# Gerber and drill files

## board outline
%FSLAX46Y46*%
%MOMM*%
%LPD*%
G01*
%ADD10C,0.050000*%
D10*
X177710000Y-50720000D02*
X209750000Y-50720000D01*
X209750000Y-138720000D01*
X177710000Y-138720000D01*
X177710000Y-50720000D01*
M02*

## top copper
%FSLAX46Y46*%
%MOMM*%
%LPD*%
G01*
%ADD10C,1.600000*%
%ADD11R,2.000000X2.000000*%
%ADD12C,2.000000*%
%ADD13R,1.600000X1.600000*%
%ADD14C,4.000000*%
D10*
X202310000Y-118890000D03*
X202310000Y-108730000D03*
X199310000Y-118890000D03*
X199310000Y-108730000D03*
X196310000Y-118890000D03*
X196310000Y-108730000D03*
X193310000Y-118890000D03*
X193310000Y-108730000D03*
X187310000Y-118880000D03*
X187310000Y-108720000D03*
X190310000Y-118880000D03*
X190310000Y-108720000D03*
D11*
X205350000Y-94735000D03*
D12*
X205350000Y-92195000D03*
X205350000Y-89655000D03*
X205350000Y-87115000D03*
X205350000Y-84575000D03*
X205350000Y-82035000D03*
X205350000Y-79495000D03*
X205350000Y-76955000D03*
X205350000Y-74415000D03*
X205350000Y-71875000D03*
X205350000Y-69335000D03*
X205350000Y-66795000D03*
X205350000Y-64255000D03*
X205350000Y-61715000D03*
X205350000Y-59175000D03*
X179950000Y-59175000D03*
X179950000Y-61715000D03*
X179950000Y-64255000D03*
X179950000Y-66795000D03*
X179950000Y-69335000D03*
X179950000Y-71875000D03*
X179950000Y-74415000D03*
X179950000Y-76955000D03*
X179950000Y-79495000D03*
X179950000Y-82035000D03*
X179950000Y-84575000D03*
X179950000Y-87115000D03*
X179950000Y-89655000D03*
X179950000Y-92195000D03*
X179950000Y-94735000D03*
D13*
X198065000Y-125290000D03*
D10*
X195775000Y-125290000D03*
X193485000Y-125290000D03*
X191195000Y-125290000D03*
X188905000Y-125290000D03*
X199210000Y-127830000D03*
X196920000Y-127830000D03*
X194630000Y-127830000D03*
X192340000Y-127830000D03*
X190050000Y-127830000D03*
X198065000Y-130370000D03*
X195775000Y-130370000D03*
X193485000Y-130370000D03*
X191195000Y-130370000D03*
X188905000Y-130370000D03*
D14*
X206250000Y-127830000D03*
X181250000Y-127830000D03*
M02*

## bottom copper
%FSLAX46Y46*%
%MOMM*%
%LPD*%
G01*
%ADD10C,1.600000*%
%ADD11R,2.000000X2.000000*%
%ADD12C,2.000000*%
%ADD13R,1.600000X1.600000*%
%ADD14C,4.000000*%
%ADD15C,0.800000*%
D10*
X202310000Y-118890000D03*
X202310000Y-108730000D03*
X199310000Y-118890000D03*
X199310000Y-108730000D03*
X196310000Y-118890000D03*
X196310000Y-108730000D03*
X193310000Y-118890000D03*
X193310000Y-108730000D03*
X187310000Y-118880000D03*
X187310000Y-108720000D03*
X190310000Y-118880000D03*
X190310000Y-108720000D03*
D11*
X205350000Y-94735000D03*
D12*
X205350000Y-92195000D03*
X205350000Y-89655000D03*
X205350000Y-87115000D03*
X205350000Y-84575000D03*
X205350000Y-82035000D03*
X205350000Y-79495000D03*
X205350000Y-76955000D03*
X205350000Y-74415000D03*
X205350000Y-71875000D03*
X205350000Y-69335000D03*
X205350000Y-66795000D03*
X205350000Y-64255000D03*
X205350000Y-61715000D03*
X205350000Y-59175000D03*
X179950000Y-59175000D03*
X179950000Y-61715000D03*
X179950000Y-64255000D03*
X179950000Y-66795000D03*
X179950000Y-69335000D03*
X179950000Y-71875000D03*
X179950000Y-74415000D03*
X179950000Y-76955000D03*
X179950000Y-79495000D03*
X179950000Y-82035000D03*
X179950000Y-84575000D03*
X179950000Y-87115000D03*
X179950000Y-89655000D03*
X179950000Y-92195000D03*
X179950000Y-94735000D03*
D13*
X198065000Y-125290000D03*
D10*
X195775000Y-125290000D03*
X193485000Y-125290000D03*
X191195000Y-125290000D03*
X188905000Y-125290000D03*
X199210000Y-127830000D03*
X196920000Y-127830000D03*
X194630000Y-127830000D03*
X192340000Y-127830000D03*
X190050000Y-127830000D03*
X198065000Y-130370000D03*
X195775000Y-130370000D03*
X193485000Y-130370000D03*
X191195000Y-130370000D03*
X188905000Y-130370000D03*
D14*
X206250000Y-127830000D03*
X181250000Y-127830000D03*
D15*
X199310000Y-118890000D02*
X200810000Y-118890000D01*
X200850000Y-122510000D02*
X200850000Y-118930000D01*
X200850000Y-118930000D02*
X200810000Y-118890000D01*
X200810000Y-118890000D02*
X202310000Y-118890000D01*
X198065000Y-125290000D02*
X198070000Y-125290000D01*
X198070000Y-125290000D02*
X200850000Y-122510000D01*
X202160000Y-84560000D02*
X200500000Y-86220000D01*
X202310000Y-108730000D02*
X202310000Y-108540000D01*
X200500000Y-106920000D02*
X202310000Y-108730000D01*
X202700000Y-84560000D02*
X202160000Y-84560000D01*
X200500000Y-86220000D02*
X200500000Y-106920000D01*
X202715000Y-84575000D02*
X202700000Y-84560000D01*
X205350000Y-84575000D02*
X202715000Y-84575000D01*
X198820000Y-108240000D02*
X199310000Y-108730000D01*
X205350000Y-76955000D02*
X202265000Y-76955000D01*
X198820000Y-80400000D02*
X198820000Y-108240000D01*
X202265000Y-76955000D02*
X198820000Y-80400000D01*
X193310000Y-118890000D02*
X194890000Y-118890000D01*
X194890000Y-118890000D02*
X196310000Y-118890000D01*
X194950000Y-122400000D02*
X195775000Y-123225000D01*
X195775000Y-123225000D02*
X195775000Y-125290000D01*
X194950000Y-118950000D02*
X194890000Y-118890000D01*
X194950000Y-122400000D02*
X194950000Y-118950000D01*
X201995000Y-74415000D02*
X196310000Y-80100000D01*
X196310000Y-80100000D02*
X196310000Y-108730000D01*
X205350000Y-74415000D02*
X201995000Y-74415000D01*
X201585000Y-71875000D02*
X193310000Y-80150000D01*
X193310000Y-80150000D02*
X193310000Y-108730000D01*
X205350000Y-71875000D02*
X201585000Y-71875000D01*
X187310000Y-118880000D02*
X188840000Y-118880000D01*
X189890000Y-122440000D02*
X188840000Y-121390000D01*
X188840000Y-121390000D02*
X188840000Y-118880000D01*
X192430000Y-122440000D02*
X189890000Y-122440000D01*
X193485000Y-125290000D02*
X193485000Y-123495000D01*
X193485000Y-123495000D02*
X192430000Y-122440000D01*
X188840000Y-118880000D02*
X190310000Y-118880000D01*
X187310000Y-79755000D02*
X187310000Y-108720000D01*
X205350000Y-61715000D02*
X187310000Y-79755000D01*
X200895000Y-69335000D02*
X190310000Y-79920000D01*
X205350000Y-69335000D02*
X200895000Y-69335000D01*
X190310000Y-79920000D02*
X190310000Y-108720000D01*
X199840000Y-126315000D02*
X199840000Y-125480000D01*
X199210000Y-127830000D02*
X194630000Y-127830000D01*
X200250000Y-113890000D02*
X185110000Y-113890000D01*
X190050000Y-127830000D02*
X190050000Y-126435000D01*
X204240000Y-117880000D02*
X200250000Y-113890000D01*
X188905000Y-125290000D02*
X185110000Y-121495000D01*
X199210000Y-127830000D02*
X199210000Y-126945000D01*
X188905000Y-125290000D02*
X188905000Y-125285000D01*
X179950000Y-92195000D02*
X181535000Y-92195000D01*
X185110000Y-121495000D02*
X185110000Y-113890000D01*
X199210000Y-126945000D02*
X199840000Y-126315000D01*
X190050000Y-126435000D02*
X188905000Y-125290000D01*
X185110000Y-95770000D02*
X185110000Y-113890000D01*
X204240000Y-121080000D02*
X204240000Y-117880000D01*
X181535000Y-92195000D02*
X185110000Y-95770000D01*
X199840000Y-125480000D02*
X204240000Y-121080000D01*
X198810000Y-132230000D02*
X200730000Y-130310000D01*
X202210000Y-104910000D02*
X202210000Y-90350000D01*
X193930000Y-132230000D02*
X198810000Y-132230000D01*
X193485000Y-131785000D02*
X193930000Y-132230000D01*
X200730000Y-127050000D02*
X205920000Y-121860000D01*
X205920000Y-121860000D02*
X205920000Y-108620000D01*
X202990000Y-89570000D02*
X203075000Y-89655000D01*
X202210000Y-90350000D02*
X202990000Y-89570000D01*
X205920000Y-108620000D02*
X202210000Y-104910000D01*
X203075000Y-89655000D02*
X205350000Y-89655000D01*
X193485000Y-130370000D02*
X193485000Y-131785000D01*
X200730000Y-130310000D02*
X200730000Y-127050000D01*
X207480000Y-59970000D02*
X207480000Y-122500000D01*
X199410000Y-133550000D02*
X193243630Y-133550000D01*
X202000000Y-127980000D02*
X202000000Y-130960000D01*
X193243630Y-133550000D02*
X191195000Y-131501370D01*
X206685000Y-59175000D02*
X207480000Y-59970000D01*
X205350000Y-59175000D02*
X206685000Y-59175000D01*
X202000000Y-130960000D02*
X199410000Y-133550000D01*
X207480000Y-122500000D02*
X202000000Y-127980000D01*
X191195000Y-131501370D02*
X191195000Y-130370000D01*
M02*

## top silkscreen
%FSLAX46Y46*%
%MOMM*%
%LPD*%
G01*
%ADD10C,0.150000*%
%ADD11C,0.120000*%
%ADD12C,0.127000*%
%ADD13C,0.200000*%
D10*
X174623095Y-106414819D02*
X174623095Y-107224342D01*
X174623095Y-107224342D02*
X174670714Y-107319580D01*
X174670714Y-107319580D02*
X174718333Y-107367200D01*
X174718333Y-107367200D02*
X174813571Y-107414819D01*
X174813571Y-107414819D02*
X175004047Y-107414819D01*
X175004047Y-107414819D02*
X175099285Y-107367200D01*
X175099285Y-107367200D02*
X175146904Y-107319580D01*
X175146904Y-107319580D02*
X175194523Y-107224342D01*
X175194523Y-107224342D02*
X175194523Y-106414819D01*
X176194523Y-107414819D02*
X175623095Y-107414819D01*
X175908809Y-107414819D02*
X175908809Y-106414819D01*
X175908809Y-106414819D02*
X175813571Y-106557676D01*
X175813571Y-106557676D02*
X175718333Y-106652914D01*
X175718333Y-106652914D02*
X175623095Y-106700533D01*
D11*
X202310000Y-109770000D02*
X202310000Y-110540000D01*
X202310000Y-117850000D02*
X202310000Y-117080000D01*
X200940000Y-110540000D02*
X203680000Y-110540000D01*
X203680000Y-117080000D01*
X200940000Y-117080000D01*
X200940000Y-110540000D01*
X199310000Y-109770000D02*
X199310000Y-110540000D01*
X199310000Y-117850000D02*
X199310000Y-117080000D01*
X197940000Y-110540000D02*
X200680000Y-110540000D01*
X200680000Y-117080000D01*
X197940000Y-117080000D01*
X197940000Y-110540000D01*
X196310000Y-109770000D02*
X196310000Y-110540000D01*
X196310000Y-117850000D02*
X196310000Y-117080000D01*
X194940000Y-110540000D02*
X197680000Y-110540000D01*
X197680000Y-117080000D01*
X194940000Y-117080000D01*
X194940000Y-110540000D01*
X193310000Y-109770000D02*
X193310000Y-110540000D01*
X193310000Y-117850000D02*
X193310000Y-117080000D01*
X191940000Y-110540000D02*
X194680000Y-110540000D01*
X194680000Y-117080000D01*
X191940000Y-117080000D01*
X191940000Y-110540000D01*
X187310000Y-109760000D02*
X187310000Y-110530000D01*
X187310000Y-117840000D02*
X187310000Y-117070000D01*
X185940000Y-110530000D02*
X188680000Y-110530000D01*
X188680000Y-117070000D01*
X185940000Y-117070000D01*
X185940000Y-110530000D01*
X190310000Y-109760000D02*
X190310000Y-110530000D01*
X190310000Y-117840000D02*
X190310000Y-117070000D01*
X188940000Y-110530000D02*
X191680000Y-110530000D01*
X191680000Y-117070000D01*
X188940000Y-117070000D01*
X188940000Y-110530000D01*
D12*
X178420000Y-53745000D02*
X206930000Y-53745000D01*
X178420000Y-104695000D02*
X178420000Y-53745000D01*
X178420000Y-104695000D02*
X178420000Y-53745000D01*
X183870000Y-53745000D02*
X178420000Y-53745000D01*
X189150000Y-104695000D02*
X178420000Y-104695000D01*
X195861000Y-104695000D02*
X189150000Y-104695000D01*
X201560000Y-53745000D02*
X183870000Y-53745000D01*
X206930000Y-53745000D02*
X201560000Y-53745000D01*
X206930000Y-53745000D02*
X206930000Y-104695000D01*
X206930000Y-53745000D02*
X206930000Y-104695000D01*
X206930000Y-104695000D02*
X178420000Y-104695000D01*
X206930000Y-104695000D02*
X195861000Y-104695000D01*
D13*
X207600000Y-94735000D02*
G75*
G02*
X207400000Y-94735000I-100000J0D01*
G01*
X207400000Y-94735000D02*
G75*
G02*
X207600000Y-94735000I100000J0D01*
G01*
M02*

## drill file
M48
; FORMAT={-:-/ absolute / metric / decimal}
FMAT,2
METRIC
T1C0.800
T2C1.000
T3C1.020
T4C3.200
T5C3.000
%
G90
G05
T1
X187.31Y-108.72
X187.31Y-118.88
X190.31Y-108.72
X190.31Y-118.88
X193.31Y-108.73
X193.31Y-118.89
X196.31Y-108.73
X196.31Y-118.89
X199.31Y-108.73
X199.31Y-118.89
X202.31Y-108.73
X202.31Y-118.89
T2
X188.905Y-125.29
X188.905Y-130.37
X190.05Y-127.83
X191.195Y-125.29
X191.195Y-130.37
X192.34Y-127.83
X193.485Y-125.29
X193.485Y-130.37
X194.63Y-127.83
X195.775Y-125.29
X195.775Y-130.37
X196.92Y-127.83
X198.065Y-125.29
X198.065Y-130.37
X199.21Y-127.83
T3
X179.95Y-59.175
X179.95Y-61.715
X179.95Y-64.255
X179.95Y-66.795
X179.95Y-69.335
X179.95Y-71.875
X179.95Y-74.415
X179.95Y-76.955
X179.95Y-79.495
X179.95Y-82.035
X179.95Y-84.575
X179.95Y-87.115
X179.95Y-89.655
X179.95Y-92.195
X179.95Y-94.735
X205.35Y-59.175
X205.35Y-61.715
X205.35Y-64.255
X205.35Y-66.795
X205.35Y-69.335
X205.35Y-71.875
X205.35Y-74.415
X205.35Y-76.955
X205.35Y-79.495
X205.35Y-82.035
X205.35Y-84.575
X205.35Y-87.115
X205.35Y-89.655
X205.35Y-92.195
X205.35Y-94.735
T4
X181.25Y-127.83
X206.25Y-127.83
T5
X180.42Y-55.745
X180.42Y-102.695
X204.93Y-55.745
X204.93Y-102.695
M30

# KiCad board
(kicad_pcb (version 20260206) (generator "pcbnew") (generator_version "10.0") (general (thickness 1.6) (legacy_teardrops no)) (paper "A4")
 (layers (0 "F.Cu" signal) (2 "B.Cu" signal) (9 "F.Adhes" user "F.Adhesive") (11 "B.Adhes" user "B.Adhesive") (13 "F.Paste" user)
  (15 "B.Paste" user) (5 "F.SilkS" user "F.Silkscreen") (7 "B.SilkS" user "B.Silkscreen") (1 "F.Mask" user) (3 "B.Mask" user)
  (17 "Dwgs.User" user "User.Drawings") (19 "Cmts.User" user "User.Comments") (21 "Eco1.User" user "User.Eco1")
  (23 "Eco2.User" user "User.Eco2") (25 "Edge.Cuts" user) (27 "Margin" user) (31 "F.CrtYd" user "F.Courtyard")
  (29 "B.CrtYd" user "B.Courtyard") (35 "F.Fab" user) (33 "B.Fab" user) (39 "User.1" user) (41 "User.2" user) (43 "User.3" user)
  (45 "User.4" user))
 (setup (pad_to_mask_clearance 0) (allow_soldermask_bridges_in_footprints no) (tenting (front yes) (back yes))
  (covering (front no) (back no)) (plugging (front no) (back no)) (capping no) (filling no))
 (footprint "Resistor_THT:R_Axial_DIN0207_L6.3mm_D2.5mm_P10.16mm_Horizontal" (layer "F.Cu") (at 202.31 118.89 90)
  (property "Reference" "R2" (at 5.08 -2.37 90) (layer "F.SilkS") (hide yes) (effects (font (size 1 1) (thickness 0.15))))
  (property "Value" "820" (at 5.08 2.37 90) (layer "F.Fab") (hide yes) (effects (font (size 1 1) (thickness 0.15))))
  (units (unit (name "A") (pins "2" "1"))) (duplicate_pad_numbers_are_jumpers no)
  (fp_line (start 9.12 0) (end 8.35 0) (stroke (width 0.12) (type solid)) (layer "F.SilkS"))
  (fp_line (start 1.04 0) (end 1.81 0) (stroke (width 0.12) (type solid)) (layer "F.SilkS"))
  (fp_rect (start 1.81 -1.37) (end 8.35 1.37) (stroke (width 0.12) (type solid)) (fill no) (layer "F.SilkS"))
  (pad "1" thru_hole circle (at 0 0 90) (size 1.6 1.6) (drill 0.8) (layers "*.Cu" "*.Mask") (remove_unused_layers no) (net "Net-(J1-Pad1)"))
  (pad "2" thru_hole circle (at 10.16 0 90) (size 1.6 1.6) (drill 0.8) (layers "*.Cu" "*.Mask") (remove_unused_layers no)
   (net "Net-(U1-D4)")))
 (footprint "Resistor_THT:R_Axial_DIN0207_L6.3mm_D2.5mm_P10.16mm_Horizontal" (layer "F.Cu") (at 199.31 118.89 90)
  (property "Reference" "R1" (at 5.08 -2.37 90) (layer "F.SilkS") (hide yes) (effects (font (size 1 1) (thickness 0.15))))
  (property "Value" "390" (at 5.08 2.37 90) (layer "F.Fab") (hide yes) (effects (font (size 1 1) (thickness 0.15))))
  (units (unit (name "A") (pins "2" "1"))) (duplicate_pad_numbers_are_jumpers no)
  (fp_line (start 9.12 0) (end 8.35 0) (stroke (width 0.12) (type solid)) (layer "F.SilkS"))
  (fp_line (start 1.04 0) (end 1.81 0) (stroke (width 0.12) (type solid)) (layer "F.SilkS"))
  (fp_rect (start 1.81 -1.37) (end 8.35 1.37) (stroke (width 0.12) (type solid)) (fill no) (layer "F.SilkS"))
  (pad "1" thru_hole circle (at 0 0 90) (size 1.6 1.6) (drill 0.8) (layers "*.Cu" "*.Mask") (remove_unused_layers no) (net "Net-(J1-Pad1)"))
  (pad "2" thru_hole circle (at 10.16 0 90) (size 1.6 1.6) (drill 0.8) (layers "*.Cu" "*.Mask") (remove_unused_layers no)
   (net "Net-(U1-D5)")))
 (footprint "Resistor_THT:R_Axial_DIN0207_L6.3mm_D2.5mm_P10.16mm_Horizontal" (layer "F.Cu") (at 196.31 118.89 90)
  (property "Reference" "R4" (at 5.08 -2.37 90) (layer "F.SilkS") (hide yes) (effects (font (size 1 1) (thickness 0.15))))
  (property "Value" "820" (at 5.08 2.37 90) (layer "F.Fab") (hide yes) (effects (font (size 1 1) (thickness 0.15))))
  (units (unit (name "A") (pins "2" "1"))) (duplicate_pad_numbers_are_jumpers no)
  (fp_line (start 9.12 0) (end 8.35 0) (stroke (width 0.12) (type solid)) (layer "F.SilkS"))
  (fp_line (start 1.04 0) (end 1.81 0) (stroke (width 0.12) (type solid)) (layer "F.SilkS"))
  (fp_rect (start 1.81 -1.37) (end 8.35 1.37) (stroke (width 0.12) (type solid)) (fill no) (layer "F.SilkS"))
  (pad "1" thru_hole circle (at 0 0 90) (size 1.6 1.6) (drill 0.8) (layers "*.Cu" "*.Mask") (remove_unused_layers no) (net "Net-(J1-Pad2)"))
  (pad "2" thru_hole circle (at 10.16 0 90) (size 1.6 1.6) (drill 0.8) (layers "*.Cu" "*.Mask") (remove_unused_layers no)
   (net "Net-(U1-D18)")))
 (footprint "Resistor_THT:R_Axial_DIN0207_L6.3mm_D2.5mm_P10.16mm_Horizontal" (layer "F.Cu") (at 193.31 118.89 90)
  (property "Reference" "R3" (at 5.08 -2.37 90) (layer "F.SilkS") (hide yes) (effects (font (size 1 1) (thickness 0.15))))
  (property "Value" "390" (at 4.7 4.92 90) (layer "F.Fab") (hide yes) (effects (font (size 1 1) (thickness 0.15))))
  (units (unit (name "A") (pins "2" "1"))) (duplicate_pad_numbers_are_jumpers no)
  (fp_line (start 9.12 0) (end 8.35 0) (stroke (width 0.12) (type solid)) (layer "F.SilkS"))
  (fp_line (start 1.04 0) (end 1.81 0) (stroke (width 0.12) (type solid)) (layer "F.SilkS"))
  (fp_rect (start 1.81 -1.37) (end 8.35 1.37) (stroke (width 0.12) (type solid)) (fill no) (layer "F.SilkS"))
  (pad "1" thru_hole circle (at 0 0 90) (size 1.6 1.6) (drill 0.8) (layers "*.Cu" "*.Mask") (remove_unused_layers no) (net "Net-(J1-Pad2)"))
  (pad "2" thru_hole circle (at 10.16 0 90) (size 1.6 1.6) (drill 0.8) (layers "*.Cu" "*.Mask") (remove_unused_layers no)
   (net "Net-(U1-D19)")))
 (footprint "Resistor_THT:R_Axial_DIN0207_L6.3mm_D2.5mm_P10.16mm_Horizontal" (layer "F.Cu") (at 187.31 118.88 90)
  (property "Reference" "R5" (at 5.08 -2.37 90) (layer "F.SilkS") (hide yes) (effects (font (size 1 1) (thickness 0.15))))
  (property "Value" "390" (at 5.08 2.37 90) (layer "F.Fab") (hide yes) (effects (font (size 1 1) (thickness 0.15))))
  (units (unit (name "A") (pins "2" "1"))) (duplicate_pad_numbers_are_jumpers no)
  (fp_line (start 9.12 0) (end 8.35 0) (stroke (width 0.12) (type solid)) (layer "F.SilkS"))
  (fp_line (start 1.04 0) (end 1.81 0) (stroke (width 0.12) (type solid)) (layer "F.SilkS"))
  (fp_rect (start 1.81 -1.37) (end 8.35 1.37) (stroke (width 0.12) (type solid)) (fill no) (layer "F.SilkS"))
  (pad "1" thru_hole circle (at 0 0 90) (size 1.6 1.6) (drill 0.8) (layers "*.Cu" "*.Mask") (remove_unused_layers no) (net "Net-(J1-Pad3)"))
  (pad "2" thru_hole circle (at 10.16 0 90) (size 1.6 1.6) (drill 0.8) (layers "*.Cu" "*.Mask") (remove_unused_layers no)
   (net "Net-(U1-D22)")))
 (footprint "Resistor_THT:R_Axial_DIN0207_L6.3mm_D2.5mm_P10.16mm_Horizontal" (layer "F.Cu") (at 190.31 118.88 90)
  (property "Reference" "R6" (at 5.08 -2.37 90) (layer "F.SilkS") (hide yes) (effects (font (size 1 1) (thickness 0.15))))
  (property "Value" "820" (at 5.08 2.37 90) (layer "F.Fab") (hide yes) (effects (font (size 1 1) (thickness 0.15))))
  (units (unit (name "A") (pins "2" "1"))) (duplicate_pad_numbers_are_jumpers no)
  (fp_line (start 9.12 0) (end 8.35 0) (stroke (width 0.12) (type solid)) (layer "F.SilkS"))
  (fp_line (start 1.04 0) (end 1.81 0) (stroke (width 0.12) (type solid)) (layer "F.SilkS"))
  (fp_rect (start 1.81 -1.37) (end 8.35 1.37) (stroke (width 0.12) (type solid)) (fill no) (layer "F.SilkS"))
  (pad "1" thru_hole circle (at 0 0 90) (size 1.6 1.6) (drill 0.8) (layers "*.Cu" "*.Mask") (remove_unused_layers no) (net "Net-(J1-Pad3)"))
  (pad "2" thru_hole circle (at 10.16 0 90) (size 1.6 1.6) (drill 0.8) (layers "*.Cu" "*.Mask") (remove_unused_layers no)
   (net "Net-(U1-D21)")))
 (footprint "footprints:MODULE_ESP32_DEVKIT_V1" (layer "F.Cu") (at 192.65 79.22 180)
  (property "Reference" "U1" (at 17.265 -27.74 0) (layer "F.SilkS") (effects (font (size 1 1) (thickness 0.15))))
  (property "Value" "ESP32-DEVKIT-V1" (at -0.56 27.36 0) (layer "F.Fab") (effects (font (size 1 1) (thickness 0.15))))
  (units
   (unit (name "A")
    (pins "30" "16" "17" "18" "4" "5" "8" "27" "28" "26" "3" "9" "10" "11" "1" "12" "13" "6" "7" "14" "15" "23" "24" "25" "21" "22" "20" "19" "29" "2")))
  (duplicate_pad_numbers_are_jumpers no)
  (fp_line (start 14.23 25.475) (end -14.28 25.475) (stroke (width 0.127) (type solid)) (layer "F.SilkS"))
  (fp_line (start 14.23 -25.475) (end 14.23 25.475) (stroke (width 0.127) (type solid)) (layer "F.SilkS"))
  (fp_line (start 14.23 -25.475) (end 14.23 25.475) (stroke (width 0.127) (type solid)) (layer "F.SilkS"))
  (fp_line (start 8.78 25.475) (end 14.23 25.475) (stroke (width 0.127) (type solid)) (layer "F.SilkS"))
  (fp_line (start 3.5 -25.475) (end 14.23 -25.475) (stroke (width 0.127) (type solid)) (layer "F.SilkS"))
  (fp_line (start -3.211 -25.475) (end 3.5 -25.475) (stroke (width 0.127) (type solid)) (layer "F.SilkS"))
  (fp_line (start -8.91 25.475) (end 8.78 25.475) (stroke (width 0.127) (type solid)) (layer "F.SilkS"))
  (fp_line (start -14.28 25.475) (end -8.91 25.475) (stroke (width 0.127) (type solid)) (layer "F.SilkS"))
  (fp_line (start -14.28 25.475) (end -14.28 -25.475) (stroke (width 0.127) (type solid)) (layer "F.SilkS"))
  (fp_line (start -14.28 25.475) (end -14.28 -25.475) (stroke (width 0.127) (type solid)) (layer "F.SilkS"))
  (fp_line (start -14.28 -25.475) (end 14.23 -25.475) (stroke (width 0.127) (type solid)) (layer "F.SilkS"))
  (fp_line (start -14.28 -25.475) (end -3.211 -25.475) (stroke (width 0.127) (type solid)) (layer "F.SilkS"))
  (fp_circle (center -14.85 -15.515) (end -14.75 -15.515) (stroke (width 0.2) (type solid)) (fill no) (layer "F.SilkS"))
  (pad "" np_thru_hole circle (at -12.28 -23.475 180) (size 3 3) (drill 3) (layers "*.Cu" "*.Mask"))
  (pad "" np_thru_hole circle (at -12.28 23.475 180) (size 3 3) (drill 3) (layers "*.Cu" "*.Mask"))
  (pad "" np_thru_hole circle (at 12.23 -23.475 180) (size 3 3) (drill 3) (layers "*.Cu" "*.Mask"))
  (pad "" np_thru_hole circle (at 12.23 23.475 180) (size 3 3) (drill 3) (layers "*.Cu" "*.Mask"))
  (pad "1" thru_hole rect (at -12.7 -15.515 180) (size 2 2) (drill 1.02) (layers "*.Cu" "*.Mask") (remove_unused_layers no)
   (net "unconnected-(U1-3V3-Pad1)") (solder_mask_margin 0.102))
  (pad "2" thru_hole circle (at -12.7 -12.975 180) (size 2 2) (drill 1.02) (layers "*.Cu" "*.Mask") (remove_unused_layers no)
   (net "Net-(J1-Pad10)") (solder_mask_margin 0.102))
  (pad "3" thru_hole circle (at -12.7 -10.435 180) (size 2 2) (drill 1.02) (layers "*.Cu" "*.Mask") (remove_unused_layers no)
   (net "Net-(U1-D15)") (solder_mask_margin 0.102))
  (pad "4" thru_hole circle (at -12.7 -7.895 180) (size 2 2) (drill 1.02) (layers "*.Cu" "*.Mask") (remove_unused_layers no)
   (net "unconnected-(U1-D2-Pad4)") (solder_mask_margin 0.102))
  (pad "5" thru_hole circle (at -12.7 -5.355 180) (size 2 2) (drill 1.02) (layers "*.Cu" "*.Mask") (remove_unused_layers no)
   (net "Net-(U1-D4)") (solder_mask_margin 0.102))
  (pad "6" thru_hole circle (at -12.7 -2.815 180) (size 2 2) (drill 1.02) (layers "*.Cu" "*.Mask") (remove_unused_layers no)
   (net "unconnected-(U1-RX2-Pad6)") (solder_mask_margin 0.102))
  (pad "7" thru_hole circle (at -12.7 -0.275 180) (size 2 2) (drill 1.02) (layers "*.Cu" "*.Mask") (remove_unused_layers no)
   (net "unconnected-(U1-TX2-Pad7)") (solder_mask_margin 0.102))
  (pad "8" thru_hole circle (at -12.7 2.265 180) (size 2 2) (drill 1.02) (layers "*.Cu" "*.Mask") (remove_unused_layers no)
   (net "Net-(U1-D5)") (solder_mask_margin 0.102))
  (pad "9" thru_hole circle (at -12.7 4.805 180) (size 2 2) (drill 1.02) (layers "*.Cu" "*.Mask") (remove_unused_layers no)
   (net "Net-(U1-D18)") (solder_mask_margin 0.102))
  (pad "10" thru_hole circle (at -12.7 7.345 180) (size 2 2) (drill 1.02) (layers "*.Cu" "*.Mask") (remove_unused_layers no)
   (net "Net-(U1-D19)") (solder_mask_margin 0.102))
  (pad "11" thru_hole circle (at -12.7 9.885 180) (size 2 2) (drill 1.02) (layers "*.Cu" "*.Mask") (remove_unused_layers no)
   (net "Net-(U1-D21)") (solder_mask_margin 0.102))
  (pad "12" thru_hole circle (at -12.7 12.425 180) (size 2 2) (drill 1.02) (layers "*.Cu" "*.Mask") (remove_unused_layers no)
   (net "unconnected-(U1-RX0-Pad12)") (solder_mask_margin 0.102))
  (pad "13" thru_hole circle (at -12.7 14.965 180) (size 2 2) (drill 1.02) (layers "*.Cu" "*.Mask") (remove_unused_layers no)
   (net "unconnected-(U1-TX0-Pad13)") (solder_mask_margin 0.102))
  (pad "14" thru_hole circle (at -12.7 17.505 180) (size 2 2) (drill 1.02) (layers "*.Cu" "*.Mask") (remove_unused_layers no)
   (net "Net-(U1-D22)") (solder_mask_margin 0.102))
  (pad "15" thru_hole circle (at -12.7 20.045 180) (size 2 2) (drill 1.02) (layers "*.Cu" "*.Mask") (remove_unused_layers no)
   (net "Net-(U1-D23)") (solder_mask_margin 0.102))
  (pad "16" thru_hole circle (at 12.7 20.045 180) (size 2 2) (drill 1.02) (layers "*.Cu" "*.Mask") (remove_unused_layers no)
   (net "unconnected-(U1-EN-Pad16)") (solder_mask_margin 0.102))
  (pad "17" thru_hole circle (at 12.7 17.505 180) (size 2 2) (drill 1.02) (layers "*.Cu" "*.Mask") (remove_unused_layers no)
   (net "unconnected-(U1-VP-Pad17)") (solder_mask_margin 0.102))
  (pad "18" thru_hole circle (at 12.7 14.965 180) (size 2 2) (drill 1.02) (layers "*.Cu" "*.Mask") (remove_unused_layers no)
   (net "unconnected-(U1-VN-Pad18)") (solder_mask_margin 0.102))
  (pad "19" thru_hole circle (at 12.7 12.425 180) (size 2 2) (drill 1.02) (layers "*.Cu" "*.Mask") (remove_unused_layers no)
   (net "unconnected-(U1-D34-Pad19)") (solder_mask_margin 0.102))
  (pad "20" thru_hole circle (at 12.7 9.885 180) (size 2 2) (drill 1.02) (layers "*.Cu" "*.Mask") (remove_unused_layers no)
   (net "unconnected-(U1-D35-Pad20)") (solder_mask_margin 0.102))
  (pad "21" thru_hole circle (at 12.7 7.345 180) (size 2 2) (drill 1.02) (layers "*.Cu" "*.Mask") (remove_unused_layers no)
   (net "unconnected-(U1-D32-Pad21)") (solder_mask_margin 0.102))
  (pad "22" thru_hole circle (at 12.7 4.805 180) (size 2 2) (drill 1.02) (layers "*.Cu" "*.Mask") (remove_unused_layers no)
   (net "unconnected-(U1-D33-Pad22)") (solder_mask_margin 0.102))
  (pad "23" thru_hole circle (at 12.7 2.265 180) (size 2 2) (drill 1.02) (layers "*.Cu" "*.Mask") (remove_unused_layers no)
   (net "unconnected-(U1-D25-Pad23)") (solder_mask_margin 0.102))
  (pad "24" thru_hole circle (at 12.7 -0.275 180) (size 2 2) (drill 1.02) (layers "*.Cu" "*.Mask") (remove_unused_layers no)
   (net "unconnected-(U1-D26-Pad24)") (solder_mask_margin 0.102))
  (pad "25" thru_hole circle (at 12.7 -2.815 180) (size 2 2) (drill 1.02) (layers "*.Cu" "*.Mask") (remove_unused_layers no)
   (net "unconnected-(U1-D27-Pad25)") (solder_mask_margin 0.102))
  (pad "26" thru_hole circle (at 12.7 -5.355 180) (size 2 2) (drill 1.02) (layers "*.Cu" "*.Mask") (remove_unused_layers no)
   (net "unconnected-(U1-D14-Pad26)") (solder_mask_margin 0.102))
  (pad "27" thru_hole circle (at 12.7 -7.895 180) (size 2 2) (drill 1.02) (layers "*.Cu" "*.Mask") (remove_unused_layers no)
   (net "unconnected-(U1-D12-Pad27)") (solder_mask_margin 0.102))
  (pad "28" thru_hole circle (at 12.7 -10.435 180) (size 2 2) (drill 1.02) (layers "*.Cu" "*.Mask") (remove_unused_layers no)
   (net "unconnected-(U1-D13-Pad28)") (solder_mask_margin 0.102))
  (pad "29" thru_hole circle (at 12.7 -12.975 180) (size 2 2) (drill 1.02) (layers "*.Cu" "*.Mask") (remove_unused_layers no)
   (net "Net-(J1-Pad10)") (solder_mask_margin 0.102))
  (pad "30" thru_hole circle (at 12.7 -15.515 180) (size 2 2) (drill 1.02) (layers "*.Cu" "*.Mask") (remove_unused_layers no)
   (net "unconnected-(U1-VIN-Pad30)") (solder_mask_margin 0.102))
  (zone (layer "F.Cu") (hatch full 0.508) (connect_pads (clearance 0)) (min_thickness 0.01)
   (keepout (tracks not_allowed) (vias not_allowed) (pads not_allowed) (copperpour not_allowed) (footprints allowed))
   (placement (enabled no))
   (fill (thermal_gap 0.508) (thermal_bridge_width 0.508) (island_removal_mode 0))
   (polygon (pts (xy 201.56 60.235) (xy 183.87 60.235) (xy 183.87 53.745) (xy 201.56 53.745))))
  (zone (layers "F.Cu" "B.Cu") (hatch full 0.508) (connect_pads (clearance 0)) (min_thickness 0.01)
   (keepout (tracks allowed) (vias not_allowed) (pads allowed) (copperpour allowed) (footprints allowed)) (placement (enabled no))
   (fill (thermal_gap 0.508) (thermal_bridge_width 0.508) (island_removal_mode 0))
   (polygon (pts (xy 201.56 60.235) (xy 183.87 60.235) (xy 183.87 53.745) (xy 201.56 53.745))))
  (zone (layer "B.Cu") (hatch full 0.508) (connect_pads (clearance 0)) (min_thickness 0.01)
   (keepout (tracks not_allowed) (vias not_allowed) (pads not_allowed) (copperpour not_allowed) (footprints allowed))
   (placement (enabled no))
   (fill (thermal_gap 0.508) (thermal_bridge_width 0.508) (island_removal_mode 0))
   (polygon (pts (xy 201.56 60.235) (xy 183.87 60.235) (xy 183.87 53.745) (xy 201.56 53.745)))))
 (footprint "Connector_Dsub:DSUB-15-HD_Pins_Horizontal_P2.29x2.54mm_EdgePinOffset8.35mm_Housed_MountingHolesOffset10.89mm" (layer "B.Cu")
  (at 198.065 125.29 180)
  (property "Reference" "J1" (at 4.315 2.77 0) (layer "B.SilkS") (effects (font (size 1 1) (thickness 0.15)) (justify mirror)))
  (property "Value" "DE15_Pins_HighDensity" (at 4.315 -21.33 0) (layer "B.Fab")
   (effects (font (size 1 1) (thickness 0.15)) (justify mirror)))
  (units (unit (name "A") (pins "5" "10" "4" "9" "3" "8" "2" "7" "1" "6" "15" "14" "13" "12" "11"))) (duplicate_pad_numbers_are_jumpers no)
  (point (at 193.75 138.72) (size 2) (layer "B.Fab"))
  (pad "1" thru_hole rect (at 0 0 180) (size 1.6 1.6) (drill 1) (layers "*.Cu" "*.Mask") (remove_unused_layers no) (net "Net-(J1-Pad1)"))
  (pad "2" thru_hole circle (at 2.29 0 180) (size 1.6 1.6) (drill 1) (layers "*.Cu" "*.Mask") (remove_unused_layers no)
   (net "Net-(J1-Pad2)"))
  (pad "3" thru_hole circle (at 4.58 0 180) (size 1.6 1.6) (drill 1) (layers "*.Cu" "*.Mask") (remove_unused_layers no)
   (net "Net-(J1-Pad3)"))
  (pad "4" thru_hole circle (at 6.87 0 180) (size 1.6 1.6) (drill 1) (layers "*.Cu" "*.Mask") (remove_unused_layers no)
   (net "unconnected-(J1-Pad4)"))
  (pad "5" thru_hole circle (at 9.16 0 180) (size 1.6 1.6) (drill 1) (layers "*.Cu" "*.Mask") (remove_unused_layers no)
   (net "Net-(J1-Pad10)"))
  (pad "6" thru_hole circle (at -1.145 -2.54 180) (size 1.6 1.6) (drill 1) (layers "*.Cu" "*.Mask") (remove_unused_layers no)
   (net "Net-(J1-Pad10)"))
  (pad "7" thru_hole circle (at 1.145 -2.54 180) (size 1.6 1.6) (drill 1) (layers "*.Cu" "*.Mask") (remove_unused_layers no)
   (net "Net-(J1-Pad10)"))
  (pad "8" thru_hole circle (at 3.435 -2.54 180) (size 1.6 1.6) (drill 1) (layers "*.Cu" "*.Mask") (remove_unused_layers no)
   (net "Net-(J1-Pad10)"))
  (pad "9" thru_hole circle (at 5.725 -2.54 180) (size 1.6 1.6) (drill 1) (layers "*.Cu" "*.Mask") (remove_unused_layers no)
   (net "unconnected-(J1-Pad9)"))
  (pad "10" thru_hole circle (at 8.015 -2.54 180) (size 1.6 1.6) (drill 1) (layers "*.Cu" "*.Mask") (remove_unused_layers no)
   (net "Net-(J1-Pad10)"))
  (pad "11" thru_hole circle (at 0 -5.08 180) (size 1.6 1.6) (drill 1) (layers "*.Cu" "*.Mask") (remove_unused_layers no)
   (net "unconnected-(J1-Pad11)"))
  (pad "12" thru_hole circle (at 2.29 -5.08 180) (size 1.6 1.6) (drill 1) (layers "*.Cu" "*.Mask") (remove_unused_layers no)
   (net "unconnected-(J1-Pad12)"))
  (pad "13" thru_hole circle (at 4.58 -5.08 180) (size 1.6 1.6) (drill 1) (layers "*.Cu" "*.Mask") (remove_unused_layers no)
   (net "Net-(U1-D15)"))
  (pad "14" thru_hole circle (at 6.87 -5.08 180) (size 1.6 1.6) (drill 1) (layers "*.Cu" "*.Mask") (remove_unused_layers no)
   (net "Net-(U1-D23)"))
  (pad "15" thru_hole circle (at 9.16 -5.08 180) (size 1.6 1.6) (drill 1) (layers "*.Cu" "*.Mask") (remove_unused_layers no)
   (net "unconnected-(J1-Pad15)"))
  (pad "SH" thru_hole circle (at -8.185 -2.54 180) (size 4 4) (drill 3.2) (layers "*.Cu" "*.Mask") (remove_unused_layers no))
  (pad "SH" thru_hole circle (at 16.815 -2.54 180) (size 4 4) (drill 3.2) (layers "*.Cu" "*.Mask") (remove_unused_layers no)))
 (gr_rect (start 177.71 50.72) (end 209.75 138.72) (stroke (width 0.05) (type default)) (fill no) (layer "Edge.Cuts"))
 (segment (start 199.31 118.89) (end 200.81 118.89) (width 0.8) (layer "B.Cu") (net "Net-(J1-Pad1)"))
 (segment (start 200.85 122.51) (end 200.85 118.93) (width 0.8) (layer "B.Cu") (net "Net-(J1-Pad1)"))
 (segment (start 200.85 118.93) (end 200.81 118.89) (width 0.8) (layer "B.Cu") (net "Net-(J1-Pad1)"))
 (segment (start 200.81 118.89) (end 202.31 118.89) (width 0.8) (layer "B.Cu") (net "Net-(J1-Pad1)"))
 (segment (start 198.065 125.29) (end 198.07 125.29) (width 0.8) (layer "B.Cu") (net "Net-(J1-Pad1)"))
 (segment (start 198.07 125.29) (end 200.85 122.51) (width 0.8) (layer "B.Cu") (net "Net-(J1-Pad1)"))
 (segment (start 202.16 84.56) (end 200.5 86.22) (width 0.8) (layer "B.Cu") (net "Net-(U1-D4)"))
 (segment (start 202.31 108.73) (end 202.31 108.54) (width 0.8) (layer "B.Cu") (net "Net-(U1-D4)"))
 (segment (start 200.5 106.92) (end 202.31 108.73) (width 0.8) (layer "B.Cu") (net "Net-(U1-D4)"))
 (segment (start 202.7 84.56) (end 202.16 84.56) (width 0.8) (layer "B.Cu") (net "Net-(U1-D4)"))
 (segment (start 200.5 86.22) (end 200.5 106.92) (width 0.8) (layer "B.Cu") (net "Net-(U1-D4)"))
 (segment (start 202.715 84.575) (end 202.7 84.56) (width 0.8) (layer "B.Cu") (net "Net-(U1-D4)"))
 (segment (start 205.35 84.575) (end 202.715 84.575) (width 0.8) (layer "B.Cu") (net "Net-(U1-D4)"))
 (segment (start 198.82 108.24) (end 199.31 108.73) (width 0.8) (layer "B.Cu") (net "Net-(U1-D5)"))
 (segment (start 205.35 76.955) (end 202.265 76.955) (width 0.8) (layer "B.Cu") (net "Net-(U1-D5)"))
 (segment (start 198.82 80.4) (end 198.82 108.24) (width 0.8) (layer "B.Cu") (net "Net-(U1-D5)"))
 (segment (start 202.265 76.955) (end 198.82 80.4) (width 0.8) (layer "B.Cu") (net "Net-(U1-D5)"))
 (segment (start 193.31 118.89) (end 194.89 118.89) (width 0.8) (layer "B.Cu") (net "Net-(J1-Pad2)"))
 (segment (start 194.89 118.89) (end 196.31 118.89) (width 0.8) (layer "B.Cu") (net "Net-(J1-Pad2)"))
 (segment (start 194.95 122.4) (end 195.775 123.225) (width 0.8) (layer "B.Cu") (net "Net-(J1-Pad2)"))
 (segment (start 195.775 123.225) (end 195.775 125.29) (width 0.8) (layer "B.Cu") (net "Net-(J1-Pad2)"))
 (segment (start 194.95 118.95) (end 194.89 118.89) (width 0.8) (layer "B.Cu") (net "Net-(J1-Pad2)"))
 (segment (start 194.95 122.4) (end 194.95 118.95) (width 0.8) (layer "B.Cu") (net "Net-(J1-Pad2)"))
 (segment (start 201.995 74.415) (end 196.31 80.1) (width 0.8) (layer "B.Cu") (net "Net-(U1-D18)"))
 (segment (start 196.31 80.1) (end 196.31 108.73) (width 0.8) (layer "B.Cu") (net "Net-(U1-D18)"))
 (segment (start 205.35 74.415) (end 201.995 74.415) (width 0.8) (layer "B.Cu") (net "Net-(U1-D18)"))
 (segment (start 201.585 71.875) (end 193.31 80.15) (width 0.8) (layer "B.Cu") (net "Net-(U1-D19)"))
 (segment (start 193.31 80.15) (end 193.31 108.73) (width 0.8) (layer "B.Cu") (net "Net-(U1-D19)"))
 (segment (start 205.35 71.875) (end 201.585 71.875) (width 0.8) (layer "B.Cu") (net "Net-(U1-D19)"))
 (segment (start 187.31 118.88) (end 188.84 118.88) (width 0.8) (layer "B.Cu") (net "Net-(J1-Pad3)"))
 (segment (start 189.89 122.44) (end 188.84 121.39) (width 0.8) (layer "B.Cu") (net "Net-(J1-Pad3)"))
 (segment (start 188.84 121.39) (end 188.84 118.88) (width 0.8) (layer "B.Cu") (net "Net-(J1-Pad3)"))
 (segment (start 192.43 122.44) (end 189.89 122.44) (width 0.8) (layer "B.Cu") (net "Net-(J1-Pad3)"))
 (segment (start 193.485 125.29) (end 193.485 123.495) (width 0.8) (layer "B.Cu") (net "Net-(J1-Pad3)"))
 (segment (start 193.485 123.495) (end 192.43 122.44) (width 0.8) (layer "B.Cu") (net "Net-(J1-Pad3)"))
 (segment (start 188.84 118.88) (end 190.31 118.88) (width 0.8) (layer "B.Cu") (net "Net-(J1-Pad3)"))
 (segment (start 187.31 79.755) (end 187.31 108.72) (width 0.8) (layer "B.Cu") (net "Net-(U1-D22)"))
 (segment (start 205.35 61.715) (end 187.31 79.755) (width 0.8) (layer "B.Cu") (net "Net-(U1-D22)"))
 (segment (start 200.895 69.335) (end 190.31 79.92) (width 0.8) (layer "B.Cu") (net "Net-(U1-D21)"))
 (segment (start 205.35 69.335) (end 200.895 69.335) (width 0.8) (layer "B.Cu") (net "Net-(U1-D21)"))
 (segment (start 190.31 79.92) (end 190.31 108.72) (width 0.8) (layer "B.Cu") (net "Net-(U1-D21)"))
 (segment (start 199.84 126.315) (end 199.84 125.48) (width 0.8) (layer "B.Cu") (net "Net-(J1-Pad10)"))
 (segment (start 199.21 127.83) (end 194.63 127.83) (width 0.8) (layer "B.Cu") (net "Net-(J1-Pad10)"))
 (segment (start 200.25 113.89) (end 185.11 113.89) (width 0.8) (layer "B.Cu") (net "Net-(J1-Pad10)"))
 (segment (start 190.05 127.83) (end 190.05 126.435) (width 0.8) (layer "B.Cu") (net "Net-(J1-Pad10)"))
 (segment (start 204.24 117.88) (end 200.25 113.89) (width 0.8) (layer "B.Cu") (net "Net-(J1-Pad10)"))
 (segment (start 188.905 125.29) (end 185.11 121.495) (width 0.8) (layer "B.Cu") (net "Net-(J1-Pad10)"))
 (segment (start 199.21 127.83) (end 199.21 126.945) (width 0.8) (layer "B.Cu") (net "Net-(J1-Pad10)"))
 (segment (start 188.905 125.29) (end 188.905 125.285) (width 0.8) (layer "B.Cu") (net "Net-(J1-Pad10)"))
 (segment (start 179.95 92.195) (end 181.535 92.195) (width 0.8) (layer "B.Cu") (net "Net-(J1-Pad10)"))
 (segment (start 185.11 121.495) (end 185.11 113.89) (width 0.8) (layer "B.Cu") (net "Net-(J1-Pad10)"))
 (segment (start 199.21 126.945) (end 199.84 126.315) (width 0.8) (layer "B.Cu") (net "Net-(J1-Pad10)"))
 (segment (start 190.05 126.435) (end 188.905 125.29) (width 0.8) (layer "B.Cu") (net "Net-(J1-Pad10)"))
 (segment (start 185.11 95.77) (end 185.11 113.89) (width 0.8) (layer "B.Cu") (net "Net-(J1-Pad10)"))
 (segment (start 204.24 121.08) (end 204.24 117.88) (width 0.8) (layer "B.Cu") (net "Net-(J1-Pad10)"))
 (segment (start 181.535 92.195) (end 185.11 95.77) (width 0.8) (layer "B.Cu") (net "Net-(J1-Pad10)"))
 (segment (start 199.84 125.48) (end 204.24 121.08) (width 0.8) (layer "B.Cu") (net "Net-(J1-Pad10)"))
 (segment (start 198.81 132.23) (end 200.73 130.31) (width 0.8) (layer "B.Cu") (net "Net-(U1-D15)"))
 (segment (start 202.21 104.91) (end 202.21 90.35) (width 0.8) (layer "B.Cu") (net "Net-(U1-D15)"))
 (segment (start 193.93 132.23) (end 198.81 132.23) (width 0.8) (layer "B.Cu") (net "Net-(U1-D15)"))
 (segment (start 193.485 131.785) (end 193.93 132.23) (width 0.8) (layer "B.Cu") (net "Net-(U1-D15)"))
 (segment (start 200.73 127.05) (end 205.92 121.86) (width 0.8) (layer "B.Cu") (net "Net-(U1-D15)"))
 (segment (start 205.92 121.86) (end 205.92 108.62) (width 0.8) (layer "B.Cu") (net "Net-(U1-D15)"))
 (segment (start 202.99 89.57) (end 203.075 89.655) (width 0.8) (layer "B.Cu") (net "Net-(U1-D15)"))
 (segment (start 202.21 90.35) (end 202.99 89.57) (width 0.8) (layer "B.Cu") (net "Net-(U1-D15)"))
 (segment (start 205.92 108.62) (end 202.21 104.91) (width 0.8) (layer "B.Cu") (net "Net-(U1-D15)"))
 (segment (start 203.075 89.655) (end 205.35 89.655) (width 0.8) (layer "B.Cu") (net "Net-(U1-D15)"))
 (segment (start 193.485 130.37) (end 193.485 131.785) (width 0.8) (layer "B.Cu") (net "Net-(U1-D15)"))
 (segment (start 200.73 130.31) (end 200.73 127.05) (width 0.8) (layer "B.Cu") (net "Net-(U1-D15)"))
 (segment (start 207.48 59.97) (end 207.48 122.5) (width 0.8) (layer "B.Cu") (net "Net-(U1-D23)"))
 (segment (start 199.41 133.55) (end 193.24363 133.55) (width 0.8) (layer "B.Cu") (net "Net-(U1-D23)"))
 (segment (start 202 127.98) (end 202 130.96) (width 0.8) (layer "B.Cu") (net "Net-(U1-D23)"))
 (segment (start 193.24363 133.55) (end 191.195 131.50137) (width 0.8) (layer "B.Cu") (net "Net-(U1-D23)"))
 (segment (start 206.685 59.175) (end 207.48 59.97) (width 0.8) (layer "B.Cu") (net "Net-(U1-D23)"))
 (segment (start 205.35 59.175) (end 206.685 59.175) (width 0.8) (layer "B.Cu") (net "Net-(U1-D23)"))
 (segment (start 202 130.96) (end 199.41 133.55) (width 0.8) (layer "B.Cu") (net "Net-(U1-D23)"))
 (segment (start 207.48 122.5) (end 202 127.98) (width 0.8) (layer "B.Cu") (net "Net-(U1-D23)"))
 (segment (start 191.195 131.50137) (end 191.195 130.37) (width 0.8) (layer "B.Cu") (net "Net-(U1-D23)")))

